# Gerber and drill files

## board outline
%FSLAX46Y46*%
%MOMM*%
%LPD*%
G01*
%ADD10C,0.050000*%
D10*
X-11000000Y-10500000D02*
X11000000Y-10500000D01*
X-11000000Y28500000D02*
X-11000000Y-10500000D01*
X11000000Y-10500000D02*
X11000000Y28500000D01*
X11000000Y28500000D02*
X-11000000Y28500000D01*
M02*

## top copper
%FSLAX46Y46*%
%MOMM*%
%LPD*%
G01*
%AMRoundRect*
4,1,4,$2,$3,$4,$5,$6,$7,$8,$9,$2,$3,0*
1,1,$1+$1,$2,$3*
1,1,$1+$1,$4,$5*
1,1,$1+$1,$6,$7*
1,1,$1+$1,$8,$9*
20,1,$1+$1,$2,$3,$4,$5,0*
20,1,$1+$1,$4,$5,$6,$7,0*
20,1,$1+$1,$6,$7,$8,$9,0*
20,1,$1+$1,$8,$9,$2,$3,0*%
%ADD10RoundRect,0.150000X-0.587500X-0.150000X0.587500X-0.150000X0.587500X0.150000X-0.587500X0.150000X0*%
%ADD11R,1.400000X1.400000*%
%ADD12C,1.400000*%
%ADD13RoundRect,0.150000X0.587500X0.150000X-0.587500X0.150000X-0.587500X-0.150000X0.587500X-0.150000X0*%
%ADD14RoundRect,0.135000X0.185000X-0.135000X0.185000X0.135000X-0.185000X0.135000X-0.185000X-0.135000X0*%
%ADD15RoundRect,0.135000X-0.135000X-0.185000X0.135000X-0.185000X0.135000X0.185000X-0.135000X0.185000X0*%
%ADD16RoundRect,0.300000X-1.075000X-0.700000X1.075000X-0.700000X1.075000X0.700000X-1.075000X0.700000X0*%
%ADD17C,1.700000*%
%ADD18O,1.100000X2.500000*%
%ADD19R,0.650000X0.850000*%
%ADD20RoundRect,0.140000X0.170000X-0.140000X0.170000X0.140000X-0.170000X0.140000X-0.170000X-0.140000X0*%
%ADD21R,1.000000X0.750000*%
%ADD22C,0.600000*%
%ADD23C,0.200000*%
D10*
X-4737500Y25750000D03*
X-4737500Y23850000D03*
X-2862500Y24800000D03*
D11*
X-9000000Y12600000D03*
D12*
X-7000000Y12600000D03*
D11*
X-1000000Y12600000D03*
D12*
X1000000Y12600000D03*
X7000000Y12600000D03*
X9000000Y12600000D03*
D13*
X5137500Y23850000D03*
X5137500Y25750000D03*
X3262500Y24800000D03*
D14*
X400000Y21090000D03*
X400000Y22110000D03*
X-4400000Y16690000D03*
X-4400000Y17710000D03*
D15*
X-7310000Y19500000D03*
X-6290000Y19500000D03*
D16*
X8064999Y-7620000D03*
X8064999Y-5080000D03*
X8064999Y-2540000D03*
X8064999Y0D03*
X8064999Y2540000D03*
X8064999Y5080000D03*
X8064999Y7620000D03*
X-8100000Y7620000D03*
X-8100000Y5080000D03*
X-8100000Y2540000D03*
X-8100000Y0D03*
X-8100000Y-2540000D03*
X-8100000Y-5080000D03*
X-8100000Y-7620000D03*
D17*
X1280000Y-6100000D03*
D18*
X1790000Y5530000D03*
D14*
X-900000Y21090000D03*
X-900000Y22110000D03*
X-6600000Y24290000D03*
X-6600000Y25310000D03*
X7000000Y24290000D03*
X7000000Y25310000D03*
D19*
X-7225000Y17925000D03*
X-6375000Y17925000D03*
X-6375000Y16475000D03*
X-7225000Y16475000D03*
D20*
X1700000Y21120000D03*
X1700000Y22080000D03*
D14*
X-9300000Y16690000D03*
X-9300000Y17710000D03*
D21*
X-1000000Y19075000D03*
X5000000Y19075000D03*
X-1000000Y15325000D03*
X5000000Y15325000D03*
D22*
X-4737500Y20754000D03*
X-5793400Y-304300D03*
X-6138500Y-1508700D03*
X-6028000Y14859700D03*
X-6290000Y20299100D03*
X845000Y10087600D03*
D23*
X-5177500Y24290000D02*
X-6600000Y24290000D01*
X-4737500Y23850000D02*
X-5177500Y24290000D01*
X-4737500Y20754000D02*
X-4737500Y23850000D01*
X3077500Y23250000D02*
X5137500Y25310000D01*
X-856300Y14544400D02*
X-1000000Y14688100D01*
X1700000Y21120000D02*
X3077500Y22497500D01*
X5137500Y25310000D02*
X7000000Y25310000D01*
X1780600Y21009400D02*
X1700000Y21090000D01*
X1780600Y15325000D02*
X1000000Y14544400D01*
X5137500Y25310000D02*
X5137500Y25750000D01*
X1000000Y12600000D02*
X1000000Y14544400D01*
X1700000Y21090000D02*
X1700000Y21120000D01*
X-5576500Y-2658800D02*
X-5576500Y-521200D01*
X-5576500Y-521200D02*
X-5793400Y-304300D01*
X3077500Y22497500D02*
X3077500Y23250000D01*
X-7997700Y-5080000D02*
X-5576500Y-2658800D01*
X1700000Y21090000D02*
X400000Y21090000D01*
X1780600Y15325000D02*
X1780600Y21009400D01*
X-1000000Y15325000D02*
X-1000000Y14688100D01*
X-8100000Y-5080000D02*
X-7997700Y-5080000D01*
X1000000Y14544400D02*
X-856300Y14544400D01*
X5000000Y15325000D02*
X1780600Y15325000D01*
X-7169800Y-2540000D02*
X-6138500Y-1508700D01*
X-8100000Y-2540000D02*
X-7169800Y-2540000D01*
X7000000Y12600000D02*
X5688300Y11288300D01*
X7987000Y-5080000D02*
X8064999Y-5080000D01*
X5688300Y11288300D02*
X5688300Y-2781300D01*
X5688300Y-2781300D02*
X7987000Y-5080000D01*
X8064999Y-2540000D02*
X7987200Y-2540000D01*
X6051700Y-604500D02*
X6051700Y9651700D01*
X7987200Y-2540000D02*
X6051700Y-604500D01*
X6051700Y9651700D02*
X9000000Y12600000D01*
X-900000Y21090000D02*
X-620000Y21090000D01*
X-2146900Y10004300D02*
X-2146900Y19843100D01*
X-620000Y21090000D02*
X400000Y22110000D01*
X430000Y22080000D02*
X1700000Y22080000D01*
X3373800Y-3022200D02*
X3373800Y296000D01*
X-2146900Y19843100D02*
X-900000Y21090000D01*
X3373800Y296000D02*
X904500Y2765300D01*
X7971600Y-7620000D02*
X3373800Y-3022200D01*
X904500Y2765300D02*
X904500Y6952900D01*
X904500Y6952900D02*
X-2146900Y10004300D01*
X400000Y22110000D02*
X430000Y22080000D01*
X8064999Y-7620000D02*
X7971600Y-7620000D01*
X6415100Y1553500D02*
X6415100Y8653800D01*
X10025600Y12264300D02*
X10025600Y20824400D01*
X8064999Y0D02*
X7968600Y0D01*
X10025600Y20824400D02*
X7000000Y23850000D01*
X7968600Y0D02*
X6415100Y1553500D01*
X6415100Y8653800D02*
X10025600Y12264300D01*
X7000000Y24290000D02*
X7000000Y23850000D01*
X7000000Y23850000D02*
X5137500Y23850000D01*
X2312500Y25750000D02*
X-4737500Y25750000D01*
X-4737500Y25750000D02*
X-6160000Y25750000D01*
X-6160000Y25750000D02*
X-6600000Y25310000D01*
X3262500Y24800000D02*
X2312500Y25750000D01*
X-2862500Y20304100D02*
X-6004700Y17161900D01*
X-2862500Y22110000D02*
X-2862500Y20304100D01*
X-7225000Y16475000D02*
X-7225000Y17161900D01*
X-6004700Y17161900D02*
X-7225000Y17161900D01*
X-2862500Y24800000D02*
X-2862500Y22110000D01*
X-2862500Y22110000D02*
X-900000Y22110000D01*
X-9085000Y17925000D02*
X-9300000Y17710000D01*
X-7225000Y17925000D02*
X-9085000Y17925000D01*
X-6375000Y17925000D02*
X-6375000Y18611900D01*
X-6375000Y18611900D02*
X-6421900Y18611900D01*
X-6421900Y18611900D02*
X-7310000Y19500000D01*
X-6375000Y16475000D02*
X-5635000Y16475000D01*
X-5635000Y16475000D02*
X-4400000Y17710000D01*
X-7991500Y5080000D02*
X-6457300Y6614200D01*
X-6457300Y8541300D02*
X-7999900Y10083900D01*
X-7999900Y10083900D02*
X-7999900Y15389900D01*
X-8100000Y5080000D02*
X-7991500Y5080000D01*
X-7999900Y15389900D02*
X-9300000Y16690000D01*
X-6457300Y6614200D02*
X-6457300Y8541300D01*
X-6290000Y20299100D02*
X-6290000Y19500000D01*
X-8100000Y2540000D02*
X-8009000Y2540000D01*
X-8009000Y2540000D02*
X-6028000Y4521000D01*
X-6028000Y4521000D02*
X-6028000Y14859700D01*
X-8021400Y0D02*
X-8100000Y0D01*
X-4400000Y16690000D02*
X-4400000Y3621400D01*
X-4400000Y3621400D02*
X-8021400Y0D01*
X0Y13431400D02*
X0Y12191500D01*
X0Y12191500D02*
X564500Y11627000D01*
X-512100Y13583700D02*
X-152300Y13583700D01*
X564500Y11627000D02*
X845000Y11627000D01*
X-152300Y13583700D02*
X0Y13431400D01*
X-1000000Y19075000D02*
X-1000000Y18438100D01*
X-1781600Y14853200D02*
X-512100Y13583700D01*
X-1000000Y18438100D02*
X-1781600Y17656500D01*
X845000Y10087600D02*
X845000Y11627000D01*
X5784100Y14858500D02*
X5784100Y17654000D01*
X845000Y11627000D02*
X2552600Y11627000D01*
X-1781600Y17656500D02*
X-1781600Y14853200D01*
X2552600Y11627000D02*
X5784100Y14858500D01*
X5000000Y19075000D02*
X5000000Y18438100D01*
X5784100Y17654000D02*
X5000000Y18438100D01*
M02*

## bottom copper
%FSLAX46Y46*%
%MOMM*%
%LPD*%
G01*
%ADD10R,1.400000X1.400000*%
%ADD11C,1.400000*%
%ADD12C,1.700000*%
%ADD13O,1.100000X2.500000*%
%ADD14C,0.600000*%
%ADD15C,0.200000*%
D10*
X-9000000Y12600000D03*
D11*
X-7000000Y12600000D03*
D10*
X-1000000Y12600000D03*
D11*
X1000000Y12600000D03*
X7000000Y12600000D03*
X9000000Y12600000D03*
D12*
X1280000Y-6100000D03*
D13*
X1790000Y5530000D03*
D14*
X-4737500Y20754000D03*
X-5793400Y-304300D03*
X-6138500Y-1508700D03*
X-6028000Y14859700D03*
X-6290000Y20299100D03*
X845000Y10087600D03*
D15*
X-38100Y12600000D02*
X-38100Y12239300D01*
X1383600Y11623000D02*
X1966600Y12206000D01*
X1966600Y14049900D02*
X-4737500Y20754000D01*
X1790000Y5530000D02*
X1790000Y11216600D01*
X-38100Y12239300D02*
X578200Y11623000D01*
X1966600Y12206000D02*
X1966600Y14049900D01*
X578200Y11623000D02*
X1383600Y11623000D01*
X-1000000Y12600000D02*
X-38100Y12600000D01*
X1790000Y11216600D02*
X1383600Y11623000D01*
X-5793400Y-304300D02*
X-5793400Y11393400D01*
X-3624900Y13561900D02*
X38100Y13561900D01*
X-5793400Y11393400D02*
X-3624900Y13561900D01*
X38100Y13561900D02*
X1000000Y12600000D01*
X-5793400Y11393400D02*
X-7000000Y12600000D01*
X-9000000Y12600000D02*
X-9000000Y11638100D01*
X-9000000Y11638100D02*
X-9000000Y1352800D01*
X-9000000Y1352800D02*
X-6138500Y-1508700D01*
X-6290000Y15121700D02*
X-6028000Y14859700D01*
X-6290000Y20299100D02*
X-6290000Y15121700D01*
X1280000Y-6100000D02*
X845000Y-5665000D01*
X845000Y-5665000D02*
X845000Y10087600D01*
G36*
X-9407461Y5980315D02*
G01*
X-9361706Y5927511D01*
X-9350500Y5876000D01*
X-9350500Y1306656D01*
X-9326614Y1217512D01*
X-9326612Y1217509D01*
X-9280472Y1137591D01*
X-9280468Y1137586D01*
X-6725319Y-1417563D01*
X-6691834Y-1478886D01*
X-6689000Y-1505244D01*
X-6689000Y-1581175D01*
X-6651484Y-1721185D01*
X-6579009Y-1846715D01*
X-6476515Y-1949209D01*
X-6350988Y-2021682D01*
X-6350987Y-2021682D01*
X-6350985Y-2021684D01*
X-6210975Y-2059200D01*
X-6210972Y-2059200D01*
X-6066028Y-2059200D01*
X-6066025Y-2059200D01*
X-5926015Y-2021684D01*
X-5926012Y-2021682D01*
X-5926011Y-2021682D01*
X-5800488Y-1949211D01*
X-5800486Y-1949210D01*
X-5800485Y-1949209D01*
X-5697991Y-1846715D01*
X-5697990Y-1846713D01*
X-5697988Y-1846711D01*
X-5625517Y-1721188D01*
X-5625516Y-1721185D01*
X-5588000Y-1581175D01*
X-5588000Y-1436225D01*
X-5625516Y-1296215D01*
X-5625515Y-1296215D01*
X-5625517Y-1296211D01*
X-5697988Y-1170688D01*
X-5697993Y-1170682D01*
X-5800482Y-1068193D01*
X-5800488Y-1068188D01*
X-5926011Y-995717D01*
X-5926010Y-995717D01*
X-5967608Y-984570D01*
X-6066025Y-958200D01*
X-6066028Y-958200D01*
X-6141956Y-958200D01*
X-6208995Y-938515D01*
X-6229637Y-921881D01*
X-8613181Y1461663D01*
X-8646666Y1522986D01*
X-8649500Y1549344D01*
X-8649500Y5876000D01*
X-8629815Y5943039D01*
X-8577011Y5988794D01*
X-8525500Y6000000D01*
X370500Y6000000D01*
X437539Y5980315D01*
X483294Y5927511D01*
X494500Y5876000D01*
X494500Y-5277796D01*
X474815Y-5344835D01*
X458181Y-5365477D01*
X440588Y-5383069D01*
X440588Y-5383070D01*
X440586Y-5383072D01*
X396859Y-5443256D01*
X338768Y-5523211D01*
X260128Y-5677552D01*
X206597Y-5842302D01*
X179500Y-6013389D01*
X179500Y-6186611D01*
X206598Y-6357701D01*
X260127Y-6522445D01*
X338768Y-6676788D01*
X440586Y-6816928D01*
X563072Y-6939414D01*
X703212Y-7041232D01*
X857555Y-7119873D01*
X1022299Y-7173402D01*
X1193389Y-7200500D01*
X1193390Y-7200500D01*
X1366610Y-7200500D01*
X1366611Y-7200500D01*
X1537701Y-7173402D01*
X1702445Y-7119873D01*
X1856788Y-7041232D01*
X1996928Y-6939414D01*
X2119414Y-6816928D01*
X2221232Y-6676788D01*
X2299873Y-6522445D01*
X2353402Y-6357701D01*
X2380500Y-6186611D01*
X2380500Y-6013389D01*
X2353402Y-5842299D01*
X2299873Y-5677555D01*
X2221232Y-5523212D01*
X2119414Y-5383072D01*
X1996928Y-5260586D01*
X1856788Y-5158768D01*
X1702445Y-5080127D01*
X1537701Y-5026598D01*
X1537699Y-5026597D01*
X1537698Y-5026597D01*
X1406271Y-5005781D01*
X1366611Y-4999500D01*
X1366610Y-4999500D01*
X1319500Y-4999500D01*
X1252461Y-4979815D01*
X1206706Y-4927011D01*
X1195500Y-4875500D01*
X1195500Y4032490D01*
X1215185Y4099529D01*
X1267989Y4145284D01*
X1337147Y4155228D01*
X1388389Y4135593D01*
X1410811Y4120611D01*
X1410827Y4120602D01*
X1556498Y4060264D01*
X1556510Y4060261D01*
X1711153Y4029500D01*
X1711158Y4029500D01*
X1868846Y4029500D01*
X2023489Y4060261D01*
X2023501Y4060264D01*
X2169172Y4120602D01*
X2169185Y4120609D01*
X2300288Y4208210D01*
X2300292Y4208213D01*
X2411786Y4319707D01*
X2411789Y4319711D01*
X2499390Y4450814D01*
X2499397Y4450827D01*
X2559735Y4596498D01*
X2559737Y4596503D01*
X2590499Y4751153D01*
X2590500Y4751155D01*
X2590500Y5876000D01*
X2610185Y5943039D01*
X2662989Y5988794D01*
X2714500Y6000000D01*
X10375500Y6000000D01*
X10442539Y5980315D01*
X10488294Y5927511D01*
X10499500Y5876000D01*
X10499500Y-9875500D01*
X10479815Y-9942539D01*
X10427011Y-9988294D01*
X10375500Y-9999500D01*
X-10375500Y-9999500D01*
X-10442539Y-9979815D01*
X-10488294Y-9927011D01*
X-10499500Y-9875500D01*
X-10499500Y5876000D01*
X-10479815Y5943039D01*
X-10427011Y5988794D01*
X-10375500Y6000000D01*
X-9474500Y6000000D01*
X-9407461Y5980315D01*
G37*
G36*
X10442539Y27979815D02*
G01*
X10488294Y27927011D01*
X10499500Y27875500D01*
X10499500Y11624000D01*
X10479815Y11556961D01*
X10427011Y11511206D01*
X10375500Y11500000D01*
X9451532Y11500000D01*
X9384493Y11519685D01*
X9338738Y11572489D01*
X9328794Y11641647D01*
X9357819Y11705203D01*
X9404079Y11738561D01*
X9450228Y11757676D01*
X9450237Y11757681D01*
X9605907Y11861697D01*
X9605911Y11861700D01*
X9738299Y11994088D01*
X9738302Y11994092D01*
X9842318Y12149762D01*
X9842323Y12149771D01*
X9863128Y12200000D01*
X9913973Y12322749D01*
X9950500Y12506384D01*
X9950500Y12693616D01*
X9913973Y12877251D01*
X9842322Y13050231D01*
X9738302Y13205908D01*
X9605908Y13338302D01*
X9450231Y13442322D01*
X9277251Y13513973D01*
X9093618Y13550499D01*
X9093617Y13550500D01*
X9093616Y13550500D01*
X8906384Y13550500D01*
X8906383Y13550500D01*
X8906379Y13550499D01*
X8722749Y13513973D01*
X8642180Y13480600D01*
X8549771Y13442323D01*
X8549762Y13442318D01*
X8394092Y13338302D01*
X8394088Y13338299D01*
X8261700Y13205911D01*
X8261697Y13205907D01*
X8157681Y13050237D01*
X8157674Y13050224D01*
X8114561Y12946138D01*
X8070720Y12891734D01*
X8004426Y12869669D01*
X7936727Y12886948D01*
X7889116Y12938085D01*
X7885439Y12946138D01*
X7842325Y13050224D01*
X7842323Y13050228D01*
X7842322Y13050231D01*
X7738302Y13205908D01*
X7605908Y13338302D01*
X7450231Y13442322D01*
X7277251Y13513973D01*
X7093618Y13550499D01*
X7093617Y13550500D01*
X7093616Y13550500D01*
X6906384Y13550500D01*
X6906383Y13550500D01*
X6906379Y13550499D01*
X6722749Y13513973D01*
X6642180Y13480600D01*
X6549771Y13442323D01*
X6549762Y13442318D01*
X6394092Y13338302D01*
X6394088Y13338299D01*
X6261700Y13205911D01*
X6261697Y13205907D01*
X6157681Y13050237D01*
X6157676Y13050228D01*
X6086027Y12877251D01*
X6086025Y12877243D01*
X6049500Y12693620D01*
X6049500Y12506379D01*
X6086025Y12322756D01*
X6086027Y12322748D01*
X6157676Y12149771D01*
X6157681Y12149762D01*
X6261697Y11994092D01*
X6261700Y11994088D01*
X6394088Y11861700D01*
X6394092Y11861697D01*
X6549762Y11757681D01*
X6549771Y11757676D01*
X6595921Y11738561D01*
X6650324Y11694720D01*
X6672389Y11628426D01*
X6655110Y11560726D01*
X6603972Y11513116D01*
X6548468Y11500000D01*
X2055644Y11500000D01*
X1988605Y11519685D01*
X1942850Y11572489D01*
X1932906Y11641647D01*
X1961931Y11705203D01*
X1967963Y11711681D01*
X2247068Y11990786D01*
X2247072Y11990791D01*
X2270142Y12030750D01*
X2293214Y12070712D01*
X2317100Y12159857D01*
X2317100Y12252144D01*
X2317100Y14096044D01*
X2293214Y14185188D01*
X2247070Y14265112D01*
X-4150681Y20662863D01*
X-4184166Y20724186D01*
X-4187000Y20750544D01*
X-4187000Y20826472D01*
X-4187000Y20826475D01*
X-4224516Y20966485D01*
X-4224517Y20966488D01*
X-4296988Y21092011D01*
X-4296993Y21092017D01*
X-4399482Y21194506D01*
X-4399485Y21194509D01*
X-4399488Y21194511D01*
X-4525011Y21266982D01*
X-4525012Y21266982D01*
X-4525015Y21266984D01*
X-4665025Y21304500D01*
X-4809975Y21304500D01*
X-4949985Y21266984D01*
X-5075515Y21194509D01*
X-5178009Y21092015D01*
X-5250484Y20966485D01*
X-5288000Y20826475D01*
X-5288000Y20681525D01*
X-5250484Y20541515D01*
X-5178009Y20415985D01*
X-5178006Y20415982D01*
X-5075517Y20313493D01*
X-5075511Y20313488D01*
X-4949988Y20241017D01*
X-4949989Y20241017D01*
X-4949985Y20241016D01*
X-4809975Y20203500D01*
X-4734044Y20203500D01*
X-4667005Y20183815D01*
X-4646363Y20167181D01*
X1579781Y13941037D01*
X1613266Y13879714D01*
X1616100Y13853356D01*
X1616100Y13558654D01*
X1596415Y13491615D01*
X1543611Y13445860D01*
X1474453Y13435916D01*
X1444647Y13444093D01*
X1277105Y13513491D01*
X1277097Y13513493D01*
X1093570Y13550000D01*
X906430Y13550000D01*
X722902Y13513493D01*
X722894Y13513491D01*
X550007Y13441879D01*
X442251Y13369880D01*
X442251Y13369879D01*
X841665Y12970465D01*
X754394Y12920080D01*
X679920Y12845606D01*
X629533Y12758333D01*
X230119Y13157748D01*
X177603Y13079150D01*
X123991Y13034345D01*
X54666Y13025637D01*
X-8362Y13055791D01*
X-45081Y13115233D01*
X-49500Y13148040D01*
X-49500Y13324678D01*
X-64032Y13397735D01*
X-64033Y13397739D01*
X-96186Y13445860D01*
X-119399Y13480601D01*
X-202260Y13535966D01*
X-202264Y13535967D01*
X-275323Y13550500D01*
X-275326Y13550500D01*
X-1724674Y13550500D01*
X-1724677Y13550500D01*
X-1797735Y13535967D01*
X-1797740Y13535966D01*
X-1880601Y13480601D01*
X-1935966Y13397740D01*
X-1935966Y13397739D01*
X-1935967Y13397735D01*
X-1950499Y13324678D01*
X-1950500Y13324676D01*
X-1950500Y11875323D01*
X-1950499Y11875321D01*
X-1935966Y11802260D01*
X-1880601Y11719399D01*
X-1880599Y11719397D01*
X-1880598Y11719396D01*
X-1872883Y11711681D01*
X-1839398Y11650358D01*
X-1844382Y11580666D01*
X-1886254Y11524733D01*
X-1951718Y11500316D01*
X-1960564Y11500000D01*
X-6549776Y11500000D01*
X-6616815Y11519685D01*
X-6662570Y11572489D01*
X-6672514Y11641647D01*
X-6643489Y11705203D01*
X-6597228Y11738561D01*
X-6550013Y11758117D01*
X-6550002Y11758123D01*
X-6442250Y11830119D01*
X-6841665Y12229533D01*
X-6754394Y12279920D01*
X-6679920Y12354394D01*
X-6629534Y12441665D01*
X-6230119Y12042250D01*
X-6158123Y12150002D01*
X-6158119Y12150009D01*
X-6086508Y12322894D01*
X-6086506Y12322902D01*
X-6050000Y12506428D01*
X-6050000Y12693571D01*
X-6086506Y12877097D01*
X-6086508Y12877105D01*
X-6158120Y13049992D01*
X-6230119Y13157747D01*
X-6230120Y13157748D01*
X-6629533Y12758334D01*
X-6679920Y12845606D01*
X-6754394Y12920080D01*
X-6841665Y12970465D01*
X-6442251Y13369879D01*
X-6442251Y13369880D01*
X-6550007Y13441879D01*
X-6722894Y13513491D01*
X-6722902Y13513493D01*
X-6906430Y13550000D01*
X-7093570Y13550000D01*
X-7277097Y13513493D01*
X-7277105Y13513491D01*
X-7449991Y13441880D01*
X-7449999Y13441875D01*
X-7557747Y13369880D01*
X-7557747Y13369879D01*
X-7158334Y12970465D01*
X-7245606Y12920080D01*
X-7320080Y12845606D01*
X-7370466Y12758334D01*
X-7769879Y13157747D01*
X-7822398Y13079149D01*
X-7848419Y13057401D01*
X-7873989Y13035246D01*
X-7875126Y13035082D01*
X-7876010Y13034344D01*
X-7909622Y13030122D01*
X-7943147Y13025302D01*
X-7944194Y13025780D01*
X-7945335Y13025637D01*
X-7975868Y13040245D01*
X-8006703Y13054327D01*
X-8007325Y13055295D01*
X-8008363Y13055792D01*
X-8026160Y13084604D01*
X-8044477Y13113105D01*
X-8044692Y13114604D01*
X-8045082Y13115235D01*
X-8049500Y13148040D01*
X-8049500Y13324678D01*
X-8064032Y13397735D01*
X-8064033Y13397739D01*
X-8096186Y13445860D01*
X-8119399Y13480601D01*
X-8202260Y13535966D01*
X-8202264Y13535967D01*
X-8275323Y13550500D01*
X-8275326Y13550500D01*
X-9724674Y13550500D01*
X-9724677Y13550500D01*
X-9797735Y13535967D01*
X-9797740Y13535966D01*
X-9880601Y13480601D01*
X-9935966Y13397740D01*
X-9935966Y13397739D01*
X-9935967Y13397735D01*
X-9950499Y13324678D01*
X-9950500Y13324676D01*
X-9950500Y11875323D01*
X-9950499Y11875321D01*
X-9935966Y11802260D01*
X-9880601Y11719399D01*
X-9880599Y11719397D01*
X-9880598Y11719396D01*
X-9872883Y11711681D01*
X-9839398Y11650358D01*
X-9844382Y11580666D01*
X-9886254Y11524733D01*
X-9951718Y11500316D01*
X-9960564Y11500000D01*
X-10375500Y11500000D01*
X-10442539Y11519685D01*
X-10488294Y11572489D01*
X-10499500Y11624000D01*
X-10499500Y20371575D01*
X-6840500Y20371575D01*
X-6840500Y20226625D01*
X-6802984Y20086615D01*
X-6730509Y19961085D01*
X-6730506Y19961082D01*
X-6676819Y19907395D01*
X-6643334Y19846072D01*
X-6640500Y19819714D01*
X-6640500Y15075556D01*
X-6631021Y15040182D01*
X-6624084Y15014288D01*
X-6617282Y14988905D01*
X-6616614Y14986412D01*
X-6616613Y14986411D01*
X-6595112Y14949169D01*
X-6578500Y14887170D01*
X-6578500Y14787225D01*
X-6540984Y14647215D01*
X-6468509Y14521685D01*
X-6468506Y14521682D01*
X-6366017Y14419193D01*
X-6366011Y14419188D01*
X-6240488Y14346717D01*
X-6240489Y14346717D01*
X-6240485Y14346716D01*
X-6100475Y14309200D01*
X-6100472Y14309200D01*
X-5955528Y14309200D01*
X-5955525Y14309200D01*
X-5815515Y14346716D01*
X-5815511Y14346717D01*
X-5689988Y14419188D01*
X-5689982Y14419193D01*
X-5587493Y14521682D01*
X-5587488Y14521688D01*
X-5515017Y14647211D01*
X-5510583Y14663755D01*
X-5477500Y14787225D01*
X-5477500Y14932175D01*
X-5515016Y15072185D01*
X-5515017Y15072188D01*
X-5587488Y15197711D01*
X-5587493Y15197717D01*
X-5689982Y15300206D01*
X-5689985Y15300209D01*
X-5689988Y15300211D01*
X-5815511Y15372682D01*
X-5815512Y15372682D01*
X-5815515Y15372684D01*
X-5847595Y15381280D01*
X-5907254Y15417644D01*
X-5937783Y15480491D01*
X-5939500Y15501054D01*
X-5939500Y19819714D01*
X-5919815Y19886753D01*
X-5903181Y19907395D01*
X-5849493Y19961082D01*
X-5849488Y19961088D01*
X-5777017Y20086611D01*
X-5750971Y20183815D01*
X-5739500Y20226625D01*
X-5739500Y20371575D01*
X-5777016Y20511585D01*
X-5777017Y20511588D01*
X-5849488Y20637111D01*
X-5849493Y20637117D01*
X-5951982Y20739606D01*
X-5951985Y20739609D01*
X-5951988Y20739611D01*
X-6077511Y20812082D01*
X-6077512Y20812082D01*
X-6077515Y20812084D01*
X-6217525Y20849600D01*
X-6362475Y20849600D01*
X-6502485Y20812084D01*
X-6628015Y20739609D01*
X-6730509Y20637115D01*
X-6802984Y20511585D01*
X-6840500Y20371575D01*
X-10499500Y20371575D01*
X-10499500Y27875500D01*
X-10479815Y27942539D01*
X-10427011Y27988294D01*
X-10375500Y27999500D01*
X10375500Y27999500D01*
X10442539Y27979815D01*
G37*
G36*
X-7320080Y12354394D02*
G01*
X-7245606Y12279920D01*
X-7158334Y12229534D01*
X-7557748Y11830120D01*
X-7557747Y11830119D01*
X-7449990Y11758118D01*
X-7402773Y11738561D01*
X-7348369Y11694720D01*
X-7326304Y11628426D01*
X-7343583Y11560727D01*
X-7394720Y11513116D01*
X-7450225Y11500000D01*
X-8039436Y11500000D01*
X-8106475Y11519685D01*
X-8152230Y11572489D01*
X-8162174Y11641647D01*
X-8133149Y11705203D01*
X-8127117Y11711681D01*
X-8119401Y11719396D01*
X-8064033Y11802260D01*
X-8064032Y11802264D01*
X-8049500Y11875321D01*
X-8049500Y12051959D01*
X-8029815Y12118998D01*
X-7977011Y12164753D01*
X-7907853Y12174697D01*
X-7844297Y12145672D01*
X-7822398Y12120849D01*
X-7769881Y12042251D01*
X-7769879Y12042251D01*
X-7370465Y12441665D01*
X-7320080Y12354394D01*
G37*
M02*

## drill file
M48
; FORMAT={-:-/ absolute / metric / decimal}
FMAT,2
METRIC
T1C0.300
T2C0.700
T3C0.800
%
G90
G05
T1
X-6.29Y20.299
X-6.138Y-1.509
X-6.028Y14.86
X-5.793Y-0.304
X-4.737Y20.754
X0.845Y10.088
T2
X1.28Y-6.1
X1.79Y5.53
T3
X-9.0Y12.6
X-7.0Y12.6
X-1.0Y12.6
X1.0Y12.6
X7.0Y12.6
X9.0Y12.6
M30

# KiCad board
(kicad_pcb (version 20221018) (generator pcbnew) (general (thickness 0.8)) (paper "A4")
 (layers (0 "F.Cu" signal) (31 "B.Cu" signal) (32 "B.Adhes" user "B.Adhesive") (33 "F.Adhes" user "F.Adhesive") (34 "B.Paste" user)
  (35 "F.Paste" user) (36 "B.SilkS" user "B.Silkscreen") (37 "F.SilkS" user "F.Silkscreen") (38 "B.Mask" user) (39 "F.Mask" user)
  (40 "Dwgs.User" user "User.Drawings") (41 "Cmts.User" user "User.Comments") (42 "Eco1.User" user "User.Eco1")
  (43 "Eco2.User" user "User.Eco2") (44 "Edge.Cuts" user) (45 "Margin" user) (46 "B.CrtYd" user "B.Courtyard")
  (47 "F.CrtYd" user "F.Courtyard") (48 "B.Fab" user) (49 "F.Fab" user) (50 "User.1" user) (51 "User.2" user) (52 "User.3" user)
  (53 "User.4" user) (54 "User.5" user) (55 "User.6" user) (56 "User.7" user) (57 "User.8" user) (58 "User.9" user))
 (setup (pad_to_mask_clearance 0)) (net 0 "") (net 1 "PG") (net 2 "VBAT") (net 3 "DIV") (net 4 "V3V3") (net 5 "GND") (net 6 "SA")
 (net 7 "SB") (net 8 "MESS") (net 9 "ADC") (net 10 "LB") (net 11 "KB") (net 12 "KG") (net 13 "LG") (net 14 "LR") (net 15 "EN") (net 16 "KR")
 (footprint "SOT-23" (layer "F.Cu") (at -3.8 -24.8)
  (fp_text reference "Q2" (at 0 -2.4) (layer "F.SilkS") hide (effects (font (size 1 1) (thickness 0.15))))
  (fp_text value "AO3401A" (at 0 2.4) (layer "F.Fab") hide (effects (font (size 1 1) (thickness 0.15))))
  (pad "1" smd roundrect (at -0.9375 -0.95) (size 1.475 0.6) (layers "F.Cu" "F.Paste" "F.Mask") (roundrect_rratio 0.25) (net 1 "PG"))
  (pad "2" smd roundrect (at -0.9375 0.95) (size 1.475 0.6) (layers "F.Cu" "F.Paste" "F.Mask") (roundrect_rratio 0.25) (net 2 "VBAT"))
  (pad "3" smd roundrect (at 0.9375 0) (size 1.475 0.6) (layers "F.Cu" "F.Paste" "F.Mask") (roundrect_rratio 0.25) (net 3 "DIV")))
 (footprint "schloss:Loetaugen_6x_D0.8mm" (layer "F.Cu") (at 0 0)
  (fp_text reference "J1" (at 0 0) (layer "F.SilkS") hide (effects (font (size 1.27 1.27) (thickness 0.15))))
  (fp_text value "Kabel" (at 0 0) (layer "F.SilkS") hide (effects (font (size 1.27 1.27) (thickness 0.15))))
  (pad "1" thru_hole rect (at -9 -12.6) (size 1.4 1.4) (drill 0.8) (layers "*.Cu" "*.Mask") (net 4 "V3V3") (thermal_bridge_angle 45))
  (pad "2" thru_hole circle (at -7 -12.6) (size 1.4 1.4) (drill 0.8) (layers "*.Cu" "*.Mask") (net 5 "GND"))
  (pad "3" thru_hole rect (at -1 -12.6) (size 1.4 1.4) (drill 0.8) (layers "*.Cu" "*.Mask") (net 2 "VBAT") (thermal_bridge_angle 45))
  (pad "4" thru_hole circle (at 1 -12.6) (size 1.4 1.4) (drill 0.8) (layers "*.Cu" "*.Mask") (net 5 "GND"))
  (pad "5" thru_hole circle (at 7 -12.6) (size 1.4 1.4) (drill 0.8) (layers "*.Cu" "*.Mask") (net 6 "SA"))
  (pad "6" thru_hole circle (at 9 -12.6) (size 1.4 1.4) (drill 0.8) (layers "*.Cu" "*.Mask") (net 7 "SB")))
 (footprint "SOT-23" (layer "F.Cu") (at 4.2 -24.8 180)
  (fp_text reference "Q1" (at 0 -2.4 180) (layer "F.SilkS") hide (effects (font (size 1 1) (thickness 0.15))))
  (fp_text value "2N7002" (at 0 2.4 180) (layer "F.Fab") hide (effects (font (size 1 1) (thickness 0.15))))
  (pad "1" smd roundrect (at -0.9375 -0.95 180) (size 1.475 0.6) (layers "F.Cu" "F.Paste" "F.Mask") (roundrect_rratio 0.25) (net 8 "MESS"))
  (pad "2" smd roundrect (at -0.9375 0.95 180) (size 1.475 0.6) (layers "F.Cu" "F.Paste" "F.Mask") (roundrect_rratio 0.25) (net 5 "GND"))
  (pad "3" smd roundrect (at 0.9375 0 180) (size 1.475 0.6) (layers "F.Cu" "F.Paste" "F.Mask") (roundrect_rratio 0.25) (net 1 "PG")))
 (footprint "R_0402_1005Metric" (layer "F.Cu") (at 0.4 -21.6 90)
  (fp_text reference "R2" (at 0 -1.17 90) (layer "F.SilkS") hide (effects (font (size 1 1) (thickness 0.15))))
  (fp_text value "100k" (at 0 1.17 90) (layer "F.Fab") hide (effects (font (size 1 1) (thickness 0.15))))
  (pad "1" smd roundrect (at -0.51 0 90) (size 0.54 0.64) (layers "F.Cu" "F.Paste" "F.Mask") (roundrect_rratio 0.25) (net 5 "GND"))
  (pad "2" smd roundrect (at 0.51 0 90) (size 0.54 0.64) (layers "F.Cu" "F.Paste" "F.Mask") (roundrect_rratio 0.25) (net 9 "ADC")))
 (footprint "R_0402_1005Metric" (layer "F.Cu") (at -4.4 -17.2 90)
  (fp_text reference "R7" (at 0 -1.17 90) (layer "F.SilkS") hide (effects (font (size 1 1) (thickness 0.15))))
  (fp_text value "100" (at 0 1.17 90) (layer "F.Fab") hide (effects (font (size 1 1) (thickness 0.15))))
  (pad "1" smd roundrect (at -0.51 0 90) (size 0.54 0.64) (layers "F.Cu" "F.Paste" "F.Mask") (roundrect_rratio 0.25) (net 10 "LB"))
  (pad "2" smd roundrect (at 0.51 0 90) (size 0.54 0.64) (layers "F.Cu" "F.Paste" "F.Mask") (roundrect_rratio 0.25) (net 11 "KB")))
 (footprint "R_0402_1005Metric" (layer "F.Cu") (at -6.8 -19.5)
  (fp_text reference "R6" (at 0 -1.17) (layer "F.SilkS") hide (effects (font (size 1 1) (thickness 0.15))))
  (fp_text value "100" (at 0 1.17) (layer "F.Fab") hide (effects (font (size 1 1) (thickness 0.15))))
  (pad "1" smd roundrect (at -0.51 0) (size 0.54 0.64) (layers "F.Cu" "F.Paste" "F.Mask") (roundrect_rratio 0.25) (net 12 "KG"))
  (pad "2" smd roundrect (at 0.51 0) (size 0.54 0.64) (layers "F.Cu" "F.Paste" "F.Mask") (roundrect_rratio 0.25) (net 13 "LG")))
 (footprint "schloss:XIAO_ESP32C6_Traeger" (layer "F.Cu") (at 0 0)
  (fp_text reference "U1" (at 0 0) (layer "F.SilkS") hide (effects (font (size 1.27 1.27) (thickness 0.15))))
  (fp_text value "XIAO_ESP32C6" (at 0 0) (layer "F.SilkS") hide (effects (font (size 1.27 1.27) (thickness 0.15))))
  (pad "1" smd roundrect (at 8.064999 7.62) (size 2.75 2) (layers "F.Cu" "F.Mask") (roundrect_rratio 0.15) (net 9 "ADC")
   (thermal_bridge_angle 45))
  (pad "2" smd roundrect (at 8.064999 5.08) (size 2.75 2) (layers "F.Cu" "F.Mask") (roundrect_rratio 0.15) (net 6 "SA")
   (thermal_bridge_angle 45))
  (pad "3" smd roundrect (at 8.064999 2.54) (size 2.75 2) (layers "F.Cu" "F.Mask") (roundrect_rratio 0.15) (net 7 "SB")
   (thermal_bridge_angle 45))
  (pad "4" smd roundrect (at 8.064999 0) (size 2.75 2) (layers "F.Cu" "F.Mask") (roundrect_rratio 0.15) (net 8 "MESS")
   (thermal_bridge_angle 45))
  (pad "5" smd roundrect (at 8.064999 -2.54) (size 2.75 2) (layers "F.Cu" "F.Mask") (roundrect_rratio 0.15) (thermal_bridge_angle 45))
  (pad "6" smd roundrect (at 8.064999 -5.08) (size 2.75 2) (layers "F.Cu" "F.Mask") (roundrect_rratio 0.15) (thermal_bridge_angle 45))
  (pad "7" smd roundrect (at 8.064999 -7.62) (size 2.75 2) (layers "F.Cu" "F.Mask") (roundrect_rratio 0.15) (thermal_bridge_angle 45))
  (pad "8" smd roundrect (at -8.1 -7.62) (size 2.75 2) (layers "F.Cu" "F.Mask") (roundrect_rratio 0.15) (thermal_bridge_angle 45))
  (pad "9" smd roundrect (at -8.1 -5.08) (size 2.75 2) (layers "F.Cu" "F.Mask") (roundrect_rratio 0.15) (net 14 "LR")
   (thermal_bridge_angle 45))
  (pad "10" smd roundrect (at -8.1 -2.54) (size 2.75 2) (layers "F.Cu" "F.Mask") (roundrect_rratio 0.15) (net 13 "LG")
   (thermal_bridge_angle 45))
  (pad "11" smd roundrect (at -8.1 0) (size 2.75 2) (layers "F.Cu" "F.Mask") (roundrect_rratio 0.15) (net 10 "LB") (thermal_bridge_angle 45))
  (pad "12" smd roundrect (at -8.1 2.54) (size 2.75 2) (layers "F.Cu" "F.Mask") (roundrect_rratio 0.15) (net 4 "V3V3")
   (thermal_bridge_angle 45))
  (pad "13" smd roundrect (at -8.1 5.08) (size 2.75 2) (layers "F.Cu" "F.Mask") (roundrect_rratio 0.15) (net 5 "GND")
   (thermal_bridge_angle 45))
  (pad "14" smd roundrect (at -8.1 7.62) (size 2.75 2) (layers "F.Cu" "F.Mask") (roundrect_rratio 0.15) (thermal_bridge_angle 45))
  (pad "17" thru_hole circle (at 1.28 6.1) (size 1.7 1.7) (drill 0.7) (layers "*.Cu" "*.Mask") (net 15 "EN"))
  (pad "23" thru_hole oval (at 1.79 -5.53) (size 1.1 2.5) (drill 0.7) (layers "*.Cu" "*.Mask") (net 2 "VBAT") (thermal_bridge_angle 45)))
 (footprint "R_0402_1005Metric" (layer "F.Cu") (at -0.9 -21.6 90)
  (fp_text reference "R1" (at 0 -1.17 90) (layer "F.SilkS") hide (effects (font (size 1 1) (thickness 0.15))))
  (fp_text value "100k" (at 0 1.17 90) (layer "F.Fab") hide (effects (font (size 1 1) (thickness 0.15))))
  (pad "1" smd roundrect (at -0.51 0 90) (size 0.54 0.64) (layers "F.Cu" "F.Paste" "F.Mask") (roundrect_rratio 0.25) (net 9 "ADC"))
  (pad "2" smd roundrect (at 0.51 0 90) (size 0.54 0.64) (layers "F.Cu" "F.Paste" "F.Mask") (roundrect_rratio 0.25) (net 3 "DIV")))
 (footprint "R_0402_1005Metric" (layer "F.Cu") (at -6.6 -24.8 90)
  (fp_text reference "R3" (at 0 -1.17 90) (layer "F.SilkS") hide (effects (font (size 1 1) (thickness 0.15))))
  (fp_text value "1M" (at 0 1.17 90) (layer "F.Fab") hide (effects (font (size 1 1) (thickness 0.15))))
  (pad "1" smd roundrect (at -0.51 0 90) (size 0.54 0.64) (layers "F.Cu" "F.Paste" "F.Mask") (roundrect_rratio 0.25) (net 2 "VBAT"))
  (pad "2" smd roundrect (at 0.51 0 90) (size 0.54 0.64) (layers "F.Cu" "F.Paste" "F.Mask") (roundrect_rratio 0.25) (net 1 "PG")))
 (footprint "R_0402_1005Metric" (layer "F.Cu") (at 7 -24.8 90)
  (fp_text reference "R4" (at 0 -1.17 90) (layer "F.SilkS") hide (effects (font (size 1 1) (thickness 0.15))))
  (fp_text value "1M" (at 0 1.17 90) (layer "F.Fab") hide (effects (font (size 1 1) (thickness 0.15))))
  (pad "1" smd roundrect (at -0.51 0 90) (size 0.54 0.64) (layers "F.Cu" "F.Paste" "F.Mask") (roundrect_rratio 0.25) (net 8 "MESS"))
  (pad "2" smd roundrect (at 0.51 0 90) (size 0.54 0.64) (layers "F.Cu" "F.Paste" "F.Mask") (roundrect_rratio 0.25) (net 5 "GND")))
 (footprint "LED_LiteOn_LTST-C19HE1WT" (layer "F.Cu") (at -6.8 -17.2)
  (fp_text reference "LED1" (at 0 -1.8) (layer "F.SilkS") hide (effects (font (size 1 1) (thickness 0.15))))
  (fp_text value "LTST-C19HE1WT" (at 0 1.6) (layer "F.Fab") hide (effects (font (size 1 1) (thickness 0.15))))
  (pad "1" smd rect (at -0.425 -0.725) (size 0.65 0.85) (layers "F.Cu" "F.Paste" "F.Mask") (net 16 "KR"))
  (pad "2" smd rect (at 0.425 -0.725) (size 0.65 0.85) (layers "F.Cu" "F.Paste" "F.Mask") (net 12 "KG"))
  (pad "3" smd rect (at 0.425 0.725) (size 0.65 0.85) (layers "F.Cu" "F.Paste" "F.Mask") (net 11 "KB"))
  (pad "4" smd rect (at -0.425 0.725) (size 0.65 0.85) (layers "F.Cu" "F.Paste" "F.Mask") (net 3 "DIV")))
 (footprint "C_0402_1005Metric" (layer "F.Cu") (at 1.7 -21.6 90)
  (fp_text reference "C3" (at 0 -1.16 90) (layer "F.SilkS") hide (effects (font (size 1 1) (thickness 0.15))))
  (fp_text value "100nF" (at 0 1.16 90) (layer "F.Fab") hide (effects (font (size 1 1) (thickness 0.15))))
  (pad "1" smd roundrect (at -0.48 0 90) (size 0.56 0.62) (layers "F.Cu" "F.Paste" "F.Mask") (roundrect_rratio 0.25) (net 5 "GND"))
  (pad "2" smd roundrect (at 0.48 0 90) (size 0.56 0.62) (layers "F.Cu" "F.Paste" "F.Mask") (roundrect_rratio 0.25) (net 9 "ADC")))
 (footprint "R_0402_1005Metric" (layer "F.Cu") (at -9.3 -17.2 90)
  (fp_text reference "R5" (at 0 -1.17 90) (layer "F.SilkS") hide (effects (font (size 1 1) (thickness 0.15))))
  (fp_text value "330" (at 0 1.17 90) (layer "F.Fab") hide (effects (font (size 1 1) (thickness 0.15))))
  (pad "1" smd roundrect (at -0.51 0 90) (size 0.54 0.64) (layers "F.Cu" "F.Paste" "F.Mask") (roundrect_rratio 0.25) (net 14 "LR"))
  (pad "2" smd roundrect (at 0.51 0 90) (size 0.54 0.64) (layers "F.Cu" "F.Paste" "F.Mask") (roundrect_rratio 0.25) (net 16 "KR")))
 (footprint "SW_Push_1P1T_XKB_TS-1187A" (layer "F.Cu") (at 2 -17.2)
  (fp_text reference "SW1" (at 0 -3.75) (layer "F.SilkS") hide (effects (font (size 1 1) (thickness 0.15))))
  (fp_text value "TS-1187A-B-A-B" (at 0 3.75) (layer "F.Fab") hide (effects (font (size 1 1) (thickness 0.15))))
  (pad "1" smd rect (at -3 -1.875) (size 1 0.75) (layers "F.Cu" "F.Paste" "F.Mask") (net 15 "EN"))
  (pad "1" smd rect (at 3 -1.875) (size 1 0.75) (layers "F.Cu" "F.Paste" "F.Mask") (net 15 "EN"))
  (pad "2" smd rect (at -3 1.875) (size 1 0.75) (layers "F.Cu" "F.Paste" "F.Mask") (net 5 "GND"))
  (pad "2" smd rect (at 3 1.875) (size 1 0.75) (layers "F.Cu" "F.Paste" "F.Mask") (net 5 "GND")))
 (gr_line (start -11 10.5) (end 11 10.5) (stroke (width 0.05) (type default)) (layer "Edge.Cuts"))
 (gr_line (start -11 -28.5) (end -11 10.5) (stroke (width 0.05) (type default)) (layer "Edge.Cuts"))
 (gr_line (start 11 10.5) (end 11 -28.5) (stroke (width 0.05) (type default)) (layer "Edge.Cuts"))
 (gr_line (start 11 -28.5) (end -11 -28.5) (stroke (width 0.05) (type default)) (layer "Edge.Cuts"))
 (segment (start -5.1775 -24.29) (end -6.6 -24.29) (width 0.2) (layer "F.Cu") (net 2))
 (segment (start -4.7375 -23.85) (end -5.1775 -24.29) (width 0.2) (layer "F.Cu") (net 2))
 (segment (start -4.7375 -20.754) (end -4.7375 -23.85) (width 0.2) (layer "F.Cu") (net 2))
 (via (at -4.7375 -20.754) (size 0.6) (drill 0.3) (layers "F.Cu" "B.Cu") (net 2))
 (segment (start -0.0381 -12.6) (end -0.0381 -12.2393) (width 0.2) (layer "B.Cu") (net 2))
 (segment (start 1.3836 -11.623) (end 1.9666 -12.206) (width 0.2) (layer "B.Cu") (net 2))
 (segment (start 1.9666 -14.0499) (end -4.7375 -20.754) (width 0.2) (layer "B.Cu") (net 2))
 (segment (start 1.79 -5.53) (end 1.79 -11.2166) (width 0.2) (layer "B.Cu") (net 2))
 (segment (start -0.0381 -12.2393) (end 0.5782 -11.623) (width 0.2) (layer "B.Cu") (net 2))
 (segment (start 1.9666 -12.206) (end 1.9666 -14.0499) (width 0.2) (layer "B.Cu") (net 2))
 (segment (start 0.5782 -11.623) (end 1.3836 -11.623) (width 0.2) (layer "B.Cu") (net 2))
 (segment (start -1 -12.6) (end -0.0381 -12.6) (width 0.2) (layer "B.Cu") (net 2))
 (segment (start 1.79 -11.2166) (end 1.3836 -11.623) (width 0.2) (layer "B.Cu") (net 2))
 (segment (start 3.0775 -23.25) (end 5.1375 -25.31) (width 0.2) (layer "F.Cu") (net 5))
 (segment (start -0.8563 -14.5444) (end -1 -14.6881) (width 0.2) (layer "F.Cu") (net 5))
 (segment (start 1.7 -21.12) (end 3.0775 -22.4975) (width 0.2) (layer "F.Cu") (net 5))
 (segment (start 5.1375 -25.31) (end 7 -25.31) (width 0.2) (layer "F.Cu") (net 5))
 (segment (start 1.7806 -21.0094) (end 1.7 -21.09) (width 0.2) (layer "F.Cu") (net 5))
 (segment (start 1.7806 -15.325) (end 1 -14.5444) (width 0.2) (layer "F.Cu") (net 5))
 (segment (start 5.1375 -25.31) (end 5.1375 -25.75) (width 0.2) (layer "F.Cu") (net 5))
 (segment (start 1 -12.6) (end 1 -14.5444) (width 0.2) (layer "F.Cu") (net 5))
 (segment (start 1.7 -21.09) (end 1.7 -21.12) (width 0.2) (layer "F.Cu") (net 5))
 (segment (start -5.5765 2.6588) (end -5.5765 0.5212) (width 0.2) (layer "F.Cu") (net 5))
 (segment (start -5.5765 0.5212) (end -5.7934 0.3043) (width 0.2) (layer "F.Cu") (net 5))
 (segment (start 3.0775 -22.4975) (end 3.0775 -23.25) (width 0.2) (layer "F.Cu") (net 5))
 (segment (start -7.9977 5.08) (end -5.5765 2.6588) (width 0.2) (layer "F.Cu") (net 5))
 (segment (start 1.7 -21.09) (end 0.4 -21.09) (width 0.2) (layer "F.Cu") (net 5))
 (segment (start 1.7806 -15.325) (end 1.7806 -21.0094) (width 0.2) (layer "F.Cu") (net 5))
 (segment (start -1 -15.325) (end -1 -14.6881) (width 0.2) (layer "F.Cu") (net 5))
 (segment (start -8.1 5.08) (end -7.9977 5.08) (width 0.2) (layer "F.Cu") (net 5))
 (segment (start 1 -14.5444) (end -0.8563 -14.5444) (width 0.2) (layer "F.Cu") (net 5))
 (segment (start 5 -15.325) (end 1.7806 -15.325) (width 0.2) (layer "F.Cu") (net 5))
 (via (at -5.7934 0.3043) (size 0.6) (drill 0.3) (layers "F.Cu" "B.Cu") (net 5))
 (segment (start -5.7934 0.3043) (end -5.7934 -11.3934) (width 0.2) (layer "B.Cu") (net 5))
 (segment (start -3.6249 -13.5619) (end 0.0381 -13.5619) (width 0.2) (layer "B.Cu") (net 5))
 (segment (start -5.7934 -11.3934) (end -3.6249 -13.5619) (width 0.2) (layer "B.Cu") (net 5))
 (segment (start 0.0381 -13.5619) (end 1 -12.6) (width 0.2) (layer "B.Cu") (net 5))
 (segment (start -5.7934 -11.3934) (end -7 -12.6) (width 0.2) (layer "B.Cu") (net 5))
 (segment (start -7.1698 2.54) (end -6.1385 1.5087) (width 0.2) (layer "F.Cu") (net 4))
 (segment (start -8.1 2.54) (end -7.1698 2.54) (width 0.2) (layer "F.Cu") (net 4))
 (via (at -6.1385 1.5087) (size 0.6) (drill 0.3) (layers "F.Cu" "B.Cu") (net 4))
 (segment (start -9 -12.6) (end -9 -11.6381) (width 0.2) (layer "B.Cu") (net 4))
 (segment (start -9 -11.6381) (end -9 -1.3528) (width 0.2) (layer "B.Cu") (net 4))
 (segment (start -9 -1.3528) (end -6.1385 1.5087) (width 0.2) (layer "B.Cu") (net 4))
 (segment (start 7 -12.6) (end 5.6883 -11.2883) (width 0.2) (layer "F.Cu") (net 6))
 (segment (start 7.987 5.08) (end 8.064999 5.08) (width 0.2) (layer "F.Cu") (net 6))
 (segment (start 5.6883 -11.2883) (end 5.6883 2.7813) (width 0.2) (layer "F.Cu") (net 6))
 (segment (start 5.6883 2.7813) (end 7.987 5.08) (width 0.2) (layer "F.Cu") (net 6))
 (segment (start 8.064999 2.54) (end 7.9872 2.54) (width 0.2) (layer "F.Cu") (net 7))
 (segment (start 6.0517 0.6045) (end 6.0517 -9.6517) (width 0.2) (layer "F.Cu") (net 7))
 (segment (start 7.9872 2.54) (end 6.0517 0.6045) (width 0.2) (layer "F.Cu") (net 7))
 (segment (start 6.0517 -9.6517) (end 9 -12.6) (width 0.2) (layer "F.Cu") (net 7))
 (segment (start -0.9 -21.09) (end -0.62 -21.09) (width 0.2) (layer "F.Cu") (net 9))
 (segment (start -2.1469 -10.0043) (end -2.1469 -19.8431) (width 0.2) (layer "F.Cu") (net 9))
 (segment (start -0.62 -21.09) (end 0.4 -22.11) (width 0.2) (layer "F.Cu") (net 9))
 (segment (start 0.43 -22.08) (end 1.7 -22.08) (width 0.2) (layer "F.Cu") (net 9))
 (segment (start 3.3738 3.0222) (end 3.3738 -0.296) (width 0.2) (layer "F.Cu") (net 9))
 (segment (start -2.1469 -19.8431) (end -0.9 -21.09) (width 0.2) (layer "F.Cu") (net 9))
 (segment (start 3.3738 -0.296) (end 0.9045 -2.7653) (width 0.2) (layer "F.Cu") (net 9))
 (segment (start 7.9716 7.62) (end 3.3738 3.0222) (width 0.2) (layer "F.Cu") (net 9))
 (segment (start 0.9045 -2.7653) (end 0.9045 -6.9529) (width 0.2) (layer "F.Cu") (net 9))
 (segment (start 0.9045 -6.9529) (end -2.1469 -10.0043) (width 0.2) (layer "F.Cu") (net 9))
 (segment (start 0.4 -22.11) (end 0.43 -22.08) (width 0.2) (layer "F.Cu") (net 9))
 (segment (start 8.064999 7.62) (end 7.9716 7.62) (width 0.2) (layer "F.Cu") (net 9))
 (segment (start 6.4151 -1.5535) (end 6.4151 -8.6538) (width 0.2) (layer "F.Cu") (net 8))
 (segment (start 10.0256 -12.2643) (end 10.0256 -20.8244) (width 0.2) (layer "F.Cu") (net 8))
 (segment (start 8.064999 0) (end 7.9686 0) (width 0.2) (layer "F.Cu") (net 8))
 (segment (start 10.0256 -20.8244) (end 7 -23.85) (width 0.2) (layer "F.Cu") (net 8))
 (segment (start 7.9686 0) (end 6.4151 -1.5535) (width 0.2) (layer "F.Cu") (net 8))
 (segment (start 6.4151 -8.6538) (end 10.0256 -12.2643) (width 0.2) (layer "F.Cu") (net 8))
 (segment (start 7 -24.29) (end 7 -23.85) (width 0.2) (layer "F.Cu") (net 8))
 (segment (start 7 -23.85) (end 5.1375 -23.85) (width 0.2) (layer "F.Cu") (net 8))
 (segment (start 2.3125 -25.75) (end -4.7375 -25.75) (width 0.2) (layer "F.Cu") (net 1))
 (segment (start -4.7375 -25.75) (end -6.16 -25.75) (width 0.2) (layer "F.Cu") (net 1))
 (segment (start -6.16 -25.75) (end -6.6 -25.31) (width 0.2) (layer "F.Cu") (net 1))
 (segment (start 3.2625 -24.8) (end 2.3125 -25.75) (width 0.2) (layer "F.Cu") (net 1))
 (segment (start -2.8625 -20.3041) (end -6.0047 -17.1619) (width 0.2) (layer "F.Cu") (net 3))
 (segment (start -2.8625 -22.11) (end -2.8625 -20.3041) (width 0.2) (layer "F.Cu") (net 3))
 (segment (start -7.225 -16.475) (end -7.225 -17.1619) (width 0.2) (layer "F.Cu") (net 3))
 (segment (start -6.0047 -17.1619) (end -7.225 -17.1619) (width 0.2) (layer "F.Cu") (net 3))
 (segment (start -2.8625 -24.8) (end -2.8625 -22.11) (width 0.2) (layer "F.Cu") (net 3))
 (segment (start -2.8625 -22.11) (end -0.9 -22.11) (width 0.2) (layer "F.Cu") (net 3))
 (segment (start -9.085 -17.925) (end -9.3 -17.71) (width 0.2) (layer "F.Cu") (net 16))
 (segment (start -7.225 -17.925) (end -9.085 -17.925) (width 0.2) (layer "F.Cu") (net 16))
 (segment (start -6.375 -17.925) (end -6.375 -18.6119) (width 0.2) (layer "F.Cu") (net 12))
 (segment (start -6.375 -18.6119) (end -6.4219 -18.6119) (width 0.2) (layer "F.Cu") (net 12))
 (segment (start -6.4219 -18.6119) (end -7.31 -19.5) (width 0.2) (layer "F.Cu") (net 12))
 (segment (start -6.375 -16.475) (end -5.635 -16.475) (width 0.2) (layer "F.Cu") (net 11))
 (segment (start -5.635 -16.475) (end -4.4 -17.71) (width 0.2) (layer "F.Cu") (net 11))
 (segment (start -7.9915 -5.08) (end -6.4573 -6.6142) (width 0.2) (layer "F.Cu") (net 14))
 (segment (start -6.4573 -8.5413) (end -7.9999 -10.0839) (width 0.2) (layer "F.Cu") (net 14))
 (segment (start -7.9999 -10.0839) (end -7.9999 -15.3899) (width 0.2) (layer "F.Cu") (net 14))
 (segment (start -8.1 -5.08) (end -7.9915 -5.08) (width 0.2) (layer "F.Cu") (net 14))
 (segment (start -7.9999 -15.3899) (end -9.3 -16.69) (width 0.2) (layer "F.Cu") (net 14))
 (segment (start -6.4573 -6.6142) (end -6.4573 -8.5413) (width 0.2) (layer "F.Cu") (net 14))
 (segment (start -6.29 -20.2991) (end -6.29 -19.5) (width 0.2) (layer "F.Cu") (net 13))
 (segment (start -8.1 -2.54) (end -8.009 -2.54) (width 0.2) (layer "F.Cu") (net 13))
 (segment (start -8.009 -2.54) (end -6.028 -4.521) (width 0.2) (layer "F.Cu") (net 13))
 (segment (start -6.028 -4.521) (end -6.028 -14.8597) (width 0.2) (layer "F.Cu") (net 13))
 (via (at -6.028 -14.8597) (size 0.6) (drill 0.3) (layers "F.Cu" "B.Cu") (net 13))
 (via (at -6.29 -20.2991) (size 0.6) (drill 0.3) (layers "F.Cu" "B.Cu") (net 13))
 (segment (start -6.29 -15.1217) (end -6.028 -14.8597) (width 0.2) (layer "B.Cu") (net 13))
 (segment (start -6.29 -20.2991) (end -6.29 -15.1217) (width 0.2) (layer "B.Cu") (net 13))
 (segment (start -8.0214 0) (end -8.1 0) (width 0.2) (layer "F.Cu") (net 10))
 (segment (start -4.4 -16.69) (end -4.4 -3.6214) (width 0.2) (layer "F.Cu") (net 10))
 (segment (start -4.4 -3.6214) (end -8.0214 0) (width 0.2) (layer "F.Cu") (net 10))
 (segment (start 0 -13.4314) (end 0 -12.1915) (width 0.2) (layer "F.Cu") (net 15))
 (segment (start 0 -12.1915) (end 0.5645 -11.627) (width 0.2) (layer "F.Cu") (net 15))
 (segment (start -0.5121 -13.5837) (end -0.1523 -13.5837) (width 0.2) (layer "F.Cu") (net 15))
 (segment (start 0.5645 -11.627) (end 0.845 -11.627) (width 0.2) (layer "F.Cu") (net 15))
 (segment (start -0.1523 -13.5837) (end 0 -13.4314) (width 0.2) (layer "F.Cu") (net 15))
 (segment (start -1 -19.075) (end -1 -18.4381) (width 0.2) (layer "F.Cu") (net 15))
 (segment (start -1.7816 -14.8532) (end -0.5121 -13.5837) (width 0.2) (layer "F.Cu") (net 15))
 (segment (start -1 -18.4381) (end -1.7816 -17.6565) (width 0.2) (layer "F.Cu") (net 15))
 (segment (start 0.845 -10.0876) (end 0.845 -11.627) (width 0.2) (layer "F.Cu") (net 15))
 (segment (start 5.7841 -14.8585) (end 5.7841 -17.654) (width 0.2) (layer "F.Cu") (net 15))
 (segment (start 0.845 -11.627) (end 2.5526 -11.627) (width 0.2) (layer "F.Cu") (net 15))
 (segment (start -1.7816 -17.6565) (end -1.7816 -14.8532) (width 0.2) (layer "F.Cu") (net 15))
 (segment (start 2.5526 -11.627) (end 5.7841 -14.8585) (width 0.2) (layer "F.Cu") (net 15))
 (segment (start 5 -19.075) (end 5 -18.4381) (width 0.2) (layer "F.Cu") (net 15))
 (segment (start 5.7841 -17.654) (end 5 -18.4381) (width 0.2) (layer "F.Cu") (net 15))
 (via (at 0.845 -10.0876) (size 0.6) (drill 0.3) (layers "F.Cu" "B.Cu") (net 15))
 (segment (start 1.28 6.1) (end 0.845 5.665) (width 0.2) (layer "B.Cu") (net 15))
 (segment (start 0.845 5.665) (end 0.845 -10.0876) (width 0.2) (layer "B.Cu") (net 15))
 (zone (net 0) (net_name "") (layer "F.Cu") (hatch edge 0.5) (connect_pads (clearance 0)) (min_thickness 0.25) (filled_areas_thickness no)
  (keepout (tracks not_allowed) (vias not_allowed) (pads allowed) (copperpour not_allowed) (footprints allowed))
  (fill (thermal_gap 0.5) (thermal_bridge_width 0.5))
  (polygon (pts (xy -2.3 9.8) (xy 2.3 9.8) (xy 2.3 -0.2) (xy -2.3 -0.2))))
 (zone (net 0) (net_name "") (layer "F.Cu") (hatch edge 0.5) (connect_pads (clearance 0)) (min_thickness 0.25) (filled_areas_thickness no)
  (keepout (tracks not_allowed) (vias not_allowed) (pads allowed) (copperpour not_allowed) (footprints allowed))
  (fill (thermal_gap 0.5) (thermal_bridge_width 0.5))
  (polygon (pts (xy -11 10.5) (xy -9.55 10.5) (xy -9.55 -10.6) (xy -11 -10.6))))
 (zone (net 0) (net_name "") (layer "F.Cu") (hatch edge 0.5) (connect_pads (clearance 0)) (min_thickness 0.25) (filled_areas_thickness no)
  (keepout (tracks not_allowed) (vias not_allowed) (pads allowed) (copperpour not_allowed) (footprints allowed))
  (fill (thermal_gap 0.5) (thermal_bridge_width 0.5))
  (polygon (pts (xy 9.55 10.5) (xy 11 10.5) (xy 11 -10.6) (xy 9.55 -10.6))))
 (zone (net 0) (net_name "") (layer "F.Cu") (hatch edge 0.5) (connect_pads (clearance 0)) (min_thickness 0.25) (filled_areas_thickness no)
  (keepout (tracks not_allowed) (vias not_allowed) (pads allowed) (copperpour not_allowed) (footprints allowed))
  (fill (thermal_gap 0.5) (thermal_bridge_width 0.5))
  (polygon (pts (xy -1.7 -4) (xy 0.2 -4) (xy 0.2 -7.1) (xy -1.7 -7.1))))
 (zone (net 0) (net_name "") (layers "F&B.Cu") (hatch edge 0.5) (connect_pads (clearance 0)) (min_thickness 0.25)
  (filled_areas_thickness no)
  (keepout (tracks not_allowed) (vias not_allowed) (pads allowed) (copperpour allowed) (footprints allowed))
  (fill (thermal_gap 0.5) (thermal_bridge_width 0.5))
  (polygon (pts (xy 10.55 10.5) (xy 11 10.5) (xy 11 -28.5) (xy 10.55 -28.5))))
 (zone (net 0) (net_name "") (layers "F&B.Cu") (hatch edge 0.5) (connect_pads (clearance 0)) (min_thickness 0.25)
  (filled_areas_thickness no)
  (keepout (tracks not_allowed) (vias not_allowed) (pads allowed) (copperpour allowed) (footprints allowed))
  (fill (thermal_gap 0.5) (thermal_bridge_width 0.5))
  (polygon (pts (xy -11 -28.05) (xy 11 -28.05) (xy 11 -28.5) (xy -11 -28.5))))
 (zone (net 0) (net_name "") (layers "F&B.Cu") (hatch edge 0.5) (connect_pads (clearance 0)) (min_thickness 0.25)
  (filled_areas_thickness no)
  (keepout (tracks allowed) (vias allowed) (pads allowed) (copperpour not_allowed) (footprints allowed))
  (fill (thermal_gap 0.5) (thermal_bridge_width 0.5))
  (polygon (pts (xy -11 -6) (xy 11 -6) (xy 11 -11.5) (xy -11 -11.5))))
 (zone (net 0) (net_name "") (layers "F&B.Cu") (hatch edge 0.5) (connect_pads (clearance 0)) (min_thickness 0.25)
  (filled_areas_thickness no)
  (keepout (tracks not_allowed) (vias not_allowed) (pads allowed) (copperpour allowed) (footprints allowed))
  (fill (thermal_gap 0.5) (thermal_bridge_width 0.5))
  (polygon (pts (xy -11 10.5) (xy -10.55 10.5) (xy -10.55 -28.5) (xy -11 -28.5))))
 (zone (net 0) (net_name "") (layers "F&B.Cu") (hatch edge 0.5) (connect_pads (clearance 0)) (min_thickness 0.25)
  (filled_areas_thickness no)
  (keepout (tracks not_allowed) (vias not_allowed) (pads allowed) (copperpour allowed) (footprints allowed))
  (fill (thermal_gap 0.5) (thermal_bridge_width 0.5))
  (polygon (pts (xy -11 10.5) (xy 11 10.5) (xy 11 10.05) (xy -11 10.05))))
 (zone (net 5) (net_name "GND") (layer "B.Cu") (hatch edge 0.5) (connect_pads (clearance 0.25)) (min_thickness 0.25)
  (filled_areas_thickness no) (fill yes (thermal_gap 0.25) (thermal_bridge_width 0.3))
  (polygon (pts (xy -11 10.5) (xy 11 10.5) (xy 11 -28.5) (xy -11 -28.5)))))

